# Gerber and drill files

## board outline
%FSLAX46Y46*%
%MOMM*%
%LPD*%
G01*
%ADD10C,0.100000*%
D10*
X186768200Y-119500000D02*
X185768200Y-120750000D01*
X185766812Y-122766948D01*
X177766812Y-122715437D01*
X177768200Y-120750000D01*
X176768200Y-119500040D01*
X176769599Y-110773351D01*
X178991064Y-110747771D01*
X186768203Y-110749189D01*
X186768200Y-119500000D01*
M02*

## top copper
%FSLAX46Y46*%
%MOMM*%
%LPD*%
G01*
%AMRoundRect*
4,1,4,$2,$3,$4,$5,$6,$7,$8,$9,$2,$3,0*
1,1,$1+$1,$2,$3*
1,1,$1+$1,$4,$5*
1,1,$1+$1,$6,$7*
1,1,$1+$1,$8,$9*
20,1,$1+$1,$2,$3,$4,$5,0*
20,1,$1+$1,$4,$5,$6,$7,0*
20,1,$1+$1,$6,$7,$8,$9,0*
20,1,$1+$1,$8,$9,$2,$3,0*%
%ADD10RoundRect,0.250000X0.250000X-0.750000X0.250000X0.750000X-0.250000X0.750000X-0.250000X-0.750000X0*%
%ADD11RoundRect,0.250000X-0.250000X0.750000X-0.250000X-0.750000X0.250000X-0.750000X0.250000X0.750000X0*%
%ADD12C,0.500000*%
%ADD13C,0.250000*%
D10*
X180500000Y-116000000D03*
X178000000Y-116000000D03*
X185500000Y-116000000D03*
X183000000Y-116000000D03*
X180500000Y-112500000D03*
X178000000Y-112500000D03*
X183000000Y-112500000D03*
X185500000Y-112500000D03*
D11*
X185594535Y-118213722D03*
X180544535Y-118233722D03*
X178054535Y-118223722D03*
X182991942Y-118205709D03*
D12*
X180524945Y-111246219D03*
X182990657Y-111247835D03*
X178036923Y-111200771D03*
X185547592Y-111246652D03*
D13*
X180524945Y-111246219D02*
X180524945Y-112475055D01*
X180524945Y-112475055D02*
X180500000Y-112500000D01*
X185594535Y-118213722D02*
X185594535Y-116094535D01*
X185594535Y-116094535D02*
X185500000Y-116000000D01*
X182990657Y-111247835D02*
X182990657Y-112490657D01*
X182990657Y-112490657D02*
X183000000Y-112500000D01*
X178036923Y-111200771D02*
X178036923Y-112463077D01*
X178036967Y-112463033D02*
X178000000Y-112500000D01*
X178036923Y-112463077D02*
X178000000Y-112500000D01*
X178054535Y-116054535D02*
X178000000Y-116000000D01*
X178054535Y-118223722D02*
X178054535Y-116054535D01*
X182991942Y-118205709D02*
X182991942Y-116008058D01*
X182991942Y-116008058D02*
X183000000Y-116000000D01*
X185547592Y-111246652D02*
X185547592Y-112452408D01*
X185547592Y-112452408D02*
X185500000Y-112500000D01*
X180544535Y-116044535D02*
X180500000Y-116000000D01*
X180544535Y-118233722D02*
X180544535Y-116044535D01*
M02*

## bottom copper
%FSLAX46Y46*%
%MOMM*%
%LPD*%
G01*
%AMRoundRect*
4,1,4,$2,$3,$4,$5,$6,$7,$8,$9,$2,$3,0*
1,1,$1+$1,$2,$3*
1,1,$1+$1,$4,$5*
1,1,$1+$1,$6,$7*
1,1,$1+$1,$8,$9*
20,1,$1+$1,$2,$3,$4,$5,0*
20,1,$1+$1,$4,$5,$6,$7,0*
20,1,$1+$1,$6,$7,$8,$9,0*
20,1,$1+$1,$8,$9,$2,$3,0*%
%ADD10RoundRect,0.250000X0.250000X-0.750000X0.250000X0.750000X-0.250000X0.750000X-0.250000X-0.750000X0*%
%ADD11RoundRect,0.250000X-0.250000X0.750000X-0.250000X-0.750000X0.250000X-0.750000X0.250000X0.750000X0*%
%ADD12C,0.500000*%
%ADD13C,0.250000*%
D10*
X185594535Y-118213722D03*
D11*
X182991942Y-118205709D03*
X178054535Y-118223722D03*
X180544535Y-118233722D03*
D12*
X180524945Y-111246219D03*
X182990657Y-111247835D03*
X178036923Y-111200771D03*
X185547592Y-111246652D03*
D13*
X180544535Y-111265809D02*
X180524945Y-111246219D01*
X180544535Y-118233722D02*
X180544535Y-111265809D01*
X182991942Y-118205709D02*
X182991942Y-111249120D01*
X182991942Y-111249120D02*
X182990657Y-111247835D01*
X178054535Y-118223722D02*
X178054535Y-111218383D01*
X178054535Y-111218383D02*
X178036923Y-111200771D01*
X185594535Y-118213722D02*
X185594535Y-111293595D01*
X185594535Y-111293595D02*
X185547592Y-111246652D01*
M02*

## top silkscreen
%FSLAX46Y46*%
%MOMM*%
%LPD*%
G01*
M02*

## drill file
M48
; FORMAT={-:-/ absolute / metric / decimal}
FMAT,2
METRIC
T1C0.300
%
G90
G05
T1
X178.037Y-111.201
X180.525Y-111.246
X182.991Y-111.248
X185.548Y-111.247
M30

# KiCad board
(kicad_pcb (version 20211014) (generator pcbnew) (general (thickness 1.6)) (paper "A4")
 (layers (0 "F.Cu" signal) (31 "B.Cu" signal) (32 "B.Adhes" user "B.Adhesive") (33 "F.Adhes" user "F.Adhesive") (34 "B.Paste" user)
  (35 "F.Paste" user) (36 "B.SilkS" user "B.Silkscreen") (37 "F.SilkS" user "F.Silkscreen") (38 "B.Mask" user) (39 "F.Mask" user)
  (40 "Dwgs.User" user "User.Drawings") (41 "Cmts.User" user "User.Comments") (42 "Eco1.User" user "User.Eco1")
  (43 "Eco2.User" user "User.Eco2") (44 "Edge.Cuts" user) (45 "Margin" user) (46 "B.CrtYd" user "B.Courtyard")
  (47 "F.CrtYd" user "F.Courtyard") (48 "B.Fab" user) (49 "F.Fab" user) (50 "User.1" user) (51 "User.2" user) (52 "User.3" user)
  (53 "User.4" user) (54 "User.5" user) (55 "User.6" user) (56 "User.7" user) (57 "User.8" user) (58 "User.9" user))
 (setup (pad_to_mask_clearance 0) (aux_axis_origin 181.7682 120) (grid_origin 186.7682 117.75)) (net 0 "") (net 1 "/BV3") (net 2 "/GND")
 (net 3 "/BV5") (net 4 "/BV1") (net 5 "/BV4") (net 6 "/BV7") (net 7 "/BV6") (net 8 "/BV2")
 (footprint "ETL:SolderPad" (layer "F.Cu") (at 181.022062 116.363766 90)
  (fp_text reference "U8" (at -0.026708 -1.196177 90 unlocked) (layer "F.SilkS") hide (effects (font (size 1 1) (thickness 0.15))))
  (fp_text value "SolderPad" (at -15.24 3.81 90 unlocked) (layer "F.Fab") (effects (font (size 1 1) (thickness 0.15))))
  (pad "1" smd roundrect (at 0.363766 -0.522062 90) (size 2 1) (layers "F.Cu" "F.Paste" "F.Mask") (roundrect_rratio 0.25) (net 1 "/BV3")))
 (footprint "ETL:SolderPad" (layer "F.Cu") (at 178.986187 116.321409 90)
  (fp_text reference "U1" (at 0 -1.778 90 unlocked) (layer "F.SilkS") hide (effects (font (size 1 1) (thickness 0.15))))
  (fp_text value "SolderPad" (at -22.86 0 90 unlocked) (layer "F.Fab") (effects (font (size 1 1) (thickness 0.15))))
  (pad "1" smd roundrect (at 0.321409 -0.986187 90) (size 2 1) (layers "F.Cu" "F.Paste" "F.Mask") (roundrect_rratio 0.25) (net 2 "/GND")))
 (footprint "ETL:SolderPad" (layer "F.Cu") (at 186.528927 116.304902 90)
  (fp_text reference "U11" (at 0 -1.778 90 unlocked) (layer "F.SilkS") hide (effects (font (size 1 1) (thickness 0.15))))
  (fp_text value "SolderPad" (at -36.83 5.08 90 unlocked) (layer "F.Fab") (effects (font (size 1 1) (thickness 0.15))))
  (pad "1" smd roundrect (at 0.304902 -1.028927 90) (size 2 1) (layers "F.Cu" "F.Paste" "F.Mask") (roundrect_rratio 0.25) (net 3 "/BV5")))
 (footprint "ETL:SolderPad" (layer "F.Cu") (at 184.018714 116.290019 90)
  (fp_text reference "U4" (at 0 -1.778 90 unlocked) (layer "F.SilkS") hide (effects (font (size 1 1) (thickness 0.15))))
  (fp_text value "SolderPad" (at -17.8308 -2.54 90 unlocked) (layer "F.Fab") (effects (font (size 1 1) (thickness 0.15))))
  (pad "1" smd roundrect (at 0.290019 -1.018714 90) (size 2 1) (layers "F.Cu" "F.Paste" "F.Mask") (roundrect_rratio 0.25) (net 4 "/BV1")))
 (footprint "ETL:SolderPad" (layer "F.Cu") (at 181.579994 113.450083 90)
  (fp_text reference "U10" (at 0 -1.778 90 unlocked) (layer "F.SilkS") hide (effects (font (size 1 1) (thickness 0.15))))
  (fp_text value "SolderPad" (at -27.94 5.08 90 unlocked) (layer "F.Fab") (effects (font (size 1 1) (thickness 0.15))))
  (pad "1" smd roundrect (at 0.950083 -1.079994 90) (size 2 1) (layers "F.Cu" "F.Paste" "F.Mask") (roundrect_rratio 0.25) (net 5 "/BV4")))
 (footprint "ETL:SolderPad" (layer "F.Cu") (at 177.908088 112.445732 90)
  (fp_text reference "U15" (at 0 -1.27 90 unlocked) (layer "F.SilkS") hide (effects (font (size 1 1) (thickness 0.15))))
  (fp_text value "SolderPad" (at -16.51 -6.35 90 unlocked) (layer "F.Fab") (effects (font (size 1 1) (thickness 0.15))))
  (pad "1" smd roundrect (at -0.054268 0.091912 90) (size 2 1) (layers "F.Cu" "F.Paste" "F.Mask") (roundrect_rratio 0.25) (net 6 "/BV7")))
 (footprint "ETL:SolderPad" (layer "F.Cu") (at 184.005468 113.41404 90)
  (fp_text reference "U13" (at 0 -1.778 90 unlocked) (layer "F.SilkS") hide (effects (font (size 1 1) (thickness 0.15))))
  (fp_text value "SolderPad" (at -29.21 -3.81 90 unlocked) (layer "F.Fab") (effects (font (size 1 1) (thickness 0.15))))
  (pad "1" smd roundrect (at 0.91404 -1.005468 90) (size 2 1) (layers "F.Cu" "F.Paste" "F.Mask") (roundrect_rratio 0.25) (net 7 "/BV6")))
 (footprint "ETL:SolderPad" (layer "F.Cu") (at 186.527934 113.473547 90)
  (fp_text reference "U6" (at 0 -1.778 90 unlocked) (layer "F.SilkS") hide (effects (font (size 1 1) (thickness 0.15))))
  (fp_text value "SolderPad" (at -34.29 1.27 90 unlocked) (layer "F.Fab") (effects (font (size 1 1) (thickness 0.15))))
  (pad "1" smd roundrect (at 0.973547 -1.027934 90) (size 2 1) (layers "F.Cu" "F.Paste" "F.Mask") (roundrect_rratio 0.25) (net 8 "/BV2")))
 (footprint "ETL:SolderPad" (layer "B.Cu") (at 185.594535 118.213722 90)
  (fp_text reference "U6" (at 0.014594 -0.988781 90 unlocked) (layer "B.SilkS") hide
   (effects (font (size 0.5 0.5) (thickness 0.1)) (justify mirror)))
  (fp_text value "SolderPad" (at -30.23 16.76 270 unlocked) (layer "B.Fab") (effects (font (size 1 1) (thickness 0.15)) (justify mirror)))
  (pad "1" smd roundrect (at 0 0 90) (size 2 1) (layers "B.Cu" "B.Paste" "B.Mask") (roundrect_rratio 0.25) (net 8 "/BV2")))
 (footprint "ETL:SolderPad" (layer "B.Cu") (at 182.991942 118.205709 -90)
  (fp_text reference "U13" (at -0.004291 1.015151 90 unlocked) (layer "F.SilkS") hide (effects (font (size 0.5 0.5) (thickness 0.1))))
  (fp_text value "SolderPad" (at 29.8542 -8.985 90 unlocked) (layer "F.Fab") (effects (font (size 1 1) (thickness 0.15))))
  (pad "1" smd roundrect (at 0 0 270) (size 2 1) (layers "B.Cu" "B.Paste" "B.Mask") (roundrect_rratio 0.25) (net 7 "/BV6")))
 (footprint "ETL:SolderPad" (layer "B.Cu") (at 178.054535 118.263722 -90)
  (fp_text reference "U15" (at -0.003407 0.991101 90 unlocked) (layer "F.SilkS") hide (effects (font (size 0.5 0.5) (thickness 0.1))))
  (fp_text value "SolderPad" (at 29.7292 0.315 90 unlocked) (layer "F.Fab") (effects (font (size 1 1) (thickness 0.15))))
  (pad "1" smd roundrect (at -0.04 0 270) (size 2 1) (layers "B.Cu" "B.Paste" "B.Mask") (roundrect_rratio 0.25) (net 6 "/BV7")))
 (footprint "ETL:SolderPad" (layer "B.Cu") (at 185.594535 118.213722 -90)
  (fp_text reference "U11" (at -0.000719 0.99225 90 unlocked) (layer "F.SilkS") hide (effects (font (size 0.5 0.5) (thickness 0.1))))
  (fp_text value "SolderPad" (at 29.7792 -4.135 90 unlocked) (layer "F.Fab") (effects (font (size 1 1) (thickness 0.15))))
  (pad "1" smd roundrect (at 0 0 270) (size 2 1) (layers "F.Cu" "F.Paste" "F.Mask") (roundrect_rratio 0.25) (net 3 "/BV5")))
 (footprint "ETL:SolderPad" (layer "B.Cu") (at 180.544535 118.284522 -90)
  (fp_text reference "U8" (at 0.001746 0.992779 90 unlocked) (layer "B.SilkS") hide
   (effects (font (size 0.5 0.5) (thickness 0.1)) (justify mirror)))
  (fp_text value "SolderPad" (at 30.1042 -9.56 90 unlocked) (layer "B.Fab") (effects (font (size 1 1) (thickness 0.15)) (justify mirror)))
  (pad "1" smd roundrect (at -0.0508 0 270) (size 2 1) (layers "F.Cu" "F.Paste" "F.Mask") (roundrect_rratio 0.25) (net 1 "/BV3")))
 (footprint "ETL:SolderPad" (layer "B.Cu") (at 178.054535 118.223722 -90)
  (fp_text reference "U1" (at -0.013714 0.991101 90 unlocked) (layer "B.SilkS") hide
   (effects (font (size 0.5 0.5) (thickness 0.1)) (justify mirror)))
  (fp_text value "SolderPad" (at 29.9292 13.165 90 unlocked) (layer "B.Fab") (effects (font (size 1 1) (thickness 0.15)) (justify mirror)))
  (pad "1" smd roundrect (at 0 0 270) (size 2 1) (layers "F.Cu" "F.Paste" "F.Mask") (roundrect_rratio 0.25) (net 2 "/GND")))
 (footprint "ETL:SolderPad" (layer "B.Cu") (at 182.991942 118.205709 -90)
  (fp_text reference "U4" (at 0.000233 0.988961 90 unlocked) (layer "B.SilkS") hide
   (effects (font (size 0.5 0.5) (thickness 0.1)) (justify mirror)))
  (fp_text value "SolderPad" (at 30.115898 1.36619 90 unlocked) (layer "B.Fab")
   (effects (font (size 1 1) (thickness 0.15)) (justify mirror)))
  (pad "1" smd roundrect (at 0 0 270) (size 2 1) (layers "F.Cu" "F.Paste" "F.Mask") (roundrect_rratio 0.25) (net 4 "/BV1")))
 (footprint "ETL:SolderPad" (layer "B.Cu") (at 180.544535 118.284522 -90)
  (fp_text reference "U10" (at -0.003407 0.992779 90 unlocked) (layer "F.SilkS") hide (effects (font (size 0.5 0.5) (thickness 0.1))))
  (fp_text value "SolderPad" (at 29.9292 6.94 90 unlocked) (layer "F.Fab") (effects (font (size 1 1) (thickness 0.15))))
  (pad "1" smd roundrect (at -0.0508 0 270) (size 2 1) (layers "B.Cu" "B.Paste" "B.Mask") (roundrect_rratio 0.25) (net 5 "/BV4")))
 (gr_poly
  (pts (xy 186.7682 119.5) (xy 185.7682 120.75) (xy 185.766812 122.766948) (xy 177.766812 122.715437) (xy 177.7682 120.75)
   (xy 176.7682 119.50004) (xy 176.769599 110.773351) (xy 178.991064 110.747771) (xy 186.768203 110.749189))
  (layer "Edge.Cuts") (width 0.1) (fill none))
 (segment (start 180.524945 111.246219) (end 180.524945 112.475055) (width 0.25) (layer "F.Cu") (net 5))
 (segment (start 180.524945 112.475055) (end 180.5 112.5) (width 0.25) (layer "F.Cu") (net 5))
 (via (at 180.524945 111.246219) (size 0.5) (drill 0.3) (layers "F.Cu" "B.Cu") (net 5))
 (segment (start 180.544535 111.265809) (end 180.524945 111.246219) (width 0.25) (layer "B.Cu") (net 5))
 (segment (start 180.544535 118.233722) (end 180.544535 111.265809) (width 0.25) (layer "B.Cu") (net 5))
 (segment (start 185.594535 118.213722) (end 185.594535 116.094535) (width 0.25) (layer "F.Cu") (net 3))
 (segment (start 185.594535 116.094535) (end 185.5 116) (width 0.25) (layer "F.Cu") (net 3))
 (segment (start 182.990657 111.247835) (end 182.990657 112.490657) (width 0.25) (layer "F.Cu") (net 7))
 (segment (start 182.990657 112.490657) (end 183 112.5) (width 0.25) (layer "F.Cu") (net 7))
 (via (at 182.990657 111.247835) (size 0.5) (drill 0.3) (layers "F.Cu" "B.Cu") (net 7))
 (segment (start 182.991942 118.205709) (end 182.991942 111.24912) (width 0.25) (layer "B.Cu") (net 7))
 (segment (start 182.991942 111.24912) (end 182.990657 111.247835) (width 0.25) (layer "B.Cu") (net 7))
 (segment (start 178.036923 111.200771) (end 178.036923 112.463077) (width 0.25) (layer "F.Cu") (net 6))
 (segment (start 178.036967 112.463033) (end 178 112.5) (width 0.25) (layer "F.Cu") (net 6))
 (segment (start 178.036923 112.463077) (end 178 112.5) (width 0.25) (layer "F.Cu") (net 6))
 (via (at 178.036923 111.200771) (size 0.5) (drill 0.3) (layers "F.Cu" "B.Cu") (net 6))
 (segment (start 178.054535 118.223722) (end 178.054535 111.218383) (width 0.25) (layer "B.Cu") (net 6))
 (segment (start 178.054535 111.218383) (end 178.036923 111.200771) (width 0.25) (layer "B.Cu") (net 6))
 (segment (start 178.054535 116.054535) (end 178 116) (width 0.25) (layer "F.Cu") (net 2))
 (segment (start 178.054535 118.223722) (end 178.054535 116.054535) (width 0.25) (layer "F.Cu") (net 2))
 (segment (start 182.991942 118.205709) (end 182.991942 116.008058) (width 0.25) (layer "F.Cu") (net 4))
 (segment (start 182.991942 116.008058) (end 183 116) (width 0.25) (layer "F.Cu") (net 4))
 (segment (start 185.547592 111.246652) (end 185.547592 112.452408) (width 0.25) (layer "F.Cu") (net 8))
 (segment (start 185.547592 112.452408) (end 185.5 112.5) (width 0.25) (layer "F.Cu") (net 8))
 (via (at 185.547592 111.246652) (size 0.5) (drill 0.3) (layers "F.Cu" "B.Cu") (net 8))
 (segment (start 185.594535 118.213722) (end 185.594535 111.293595) (width 0.25) (layer "B.Cu") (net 8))
 (segment (start 185.594535 111.293595) (end 185.547592 111.246652) (width 0.25) (layer "B.Cu") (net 8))
 (segment (start 180.544535 116.044535) (end 180.5 116) (width 0.25) (layer "F.Cu") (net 1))
 (segment (start 180.544535 118.233722) (end 180.544535 116.044535) (width 0.25) (layer "F.Cu") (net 1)))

